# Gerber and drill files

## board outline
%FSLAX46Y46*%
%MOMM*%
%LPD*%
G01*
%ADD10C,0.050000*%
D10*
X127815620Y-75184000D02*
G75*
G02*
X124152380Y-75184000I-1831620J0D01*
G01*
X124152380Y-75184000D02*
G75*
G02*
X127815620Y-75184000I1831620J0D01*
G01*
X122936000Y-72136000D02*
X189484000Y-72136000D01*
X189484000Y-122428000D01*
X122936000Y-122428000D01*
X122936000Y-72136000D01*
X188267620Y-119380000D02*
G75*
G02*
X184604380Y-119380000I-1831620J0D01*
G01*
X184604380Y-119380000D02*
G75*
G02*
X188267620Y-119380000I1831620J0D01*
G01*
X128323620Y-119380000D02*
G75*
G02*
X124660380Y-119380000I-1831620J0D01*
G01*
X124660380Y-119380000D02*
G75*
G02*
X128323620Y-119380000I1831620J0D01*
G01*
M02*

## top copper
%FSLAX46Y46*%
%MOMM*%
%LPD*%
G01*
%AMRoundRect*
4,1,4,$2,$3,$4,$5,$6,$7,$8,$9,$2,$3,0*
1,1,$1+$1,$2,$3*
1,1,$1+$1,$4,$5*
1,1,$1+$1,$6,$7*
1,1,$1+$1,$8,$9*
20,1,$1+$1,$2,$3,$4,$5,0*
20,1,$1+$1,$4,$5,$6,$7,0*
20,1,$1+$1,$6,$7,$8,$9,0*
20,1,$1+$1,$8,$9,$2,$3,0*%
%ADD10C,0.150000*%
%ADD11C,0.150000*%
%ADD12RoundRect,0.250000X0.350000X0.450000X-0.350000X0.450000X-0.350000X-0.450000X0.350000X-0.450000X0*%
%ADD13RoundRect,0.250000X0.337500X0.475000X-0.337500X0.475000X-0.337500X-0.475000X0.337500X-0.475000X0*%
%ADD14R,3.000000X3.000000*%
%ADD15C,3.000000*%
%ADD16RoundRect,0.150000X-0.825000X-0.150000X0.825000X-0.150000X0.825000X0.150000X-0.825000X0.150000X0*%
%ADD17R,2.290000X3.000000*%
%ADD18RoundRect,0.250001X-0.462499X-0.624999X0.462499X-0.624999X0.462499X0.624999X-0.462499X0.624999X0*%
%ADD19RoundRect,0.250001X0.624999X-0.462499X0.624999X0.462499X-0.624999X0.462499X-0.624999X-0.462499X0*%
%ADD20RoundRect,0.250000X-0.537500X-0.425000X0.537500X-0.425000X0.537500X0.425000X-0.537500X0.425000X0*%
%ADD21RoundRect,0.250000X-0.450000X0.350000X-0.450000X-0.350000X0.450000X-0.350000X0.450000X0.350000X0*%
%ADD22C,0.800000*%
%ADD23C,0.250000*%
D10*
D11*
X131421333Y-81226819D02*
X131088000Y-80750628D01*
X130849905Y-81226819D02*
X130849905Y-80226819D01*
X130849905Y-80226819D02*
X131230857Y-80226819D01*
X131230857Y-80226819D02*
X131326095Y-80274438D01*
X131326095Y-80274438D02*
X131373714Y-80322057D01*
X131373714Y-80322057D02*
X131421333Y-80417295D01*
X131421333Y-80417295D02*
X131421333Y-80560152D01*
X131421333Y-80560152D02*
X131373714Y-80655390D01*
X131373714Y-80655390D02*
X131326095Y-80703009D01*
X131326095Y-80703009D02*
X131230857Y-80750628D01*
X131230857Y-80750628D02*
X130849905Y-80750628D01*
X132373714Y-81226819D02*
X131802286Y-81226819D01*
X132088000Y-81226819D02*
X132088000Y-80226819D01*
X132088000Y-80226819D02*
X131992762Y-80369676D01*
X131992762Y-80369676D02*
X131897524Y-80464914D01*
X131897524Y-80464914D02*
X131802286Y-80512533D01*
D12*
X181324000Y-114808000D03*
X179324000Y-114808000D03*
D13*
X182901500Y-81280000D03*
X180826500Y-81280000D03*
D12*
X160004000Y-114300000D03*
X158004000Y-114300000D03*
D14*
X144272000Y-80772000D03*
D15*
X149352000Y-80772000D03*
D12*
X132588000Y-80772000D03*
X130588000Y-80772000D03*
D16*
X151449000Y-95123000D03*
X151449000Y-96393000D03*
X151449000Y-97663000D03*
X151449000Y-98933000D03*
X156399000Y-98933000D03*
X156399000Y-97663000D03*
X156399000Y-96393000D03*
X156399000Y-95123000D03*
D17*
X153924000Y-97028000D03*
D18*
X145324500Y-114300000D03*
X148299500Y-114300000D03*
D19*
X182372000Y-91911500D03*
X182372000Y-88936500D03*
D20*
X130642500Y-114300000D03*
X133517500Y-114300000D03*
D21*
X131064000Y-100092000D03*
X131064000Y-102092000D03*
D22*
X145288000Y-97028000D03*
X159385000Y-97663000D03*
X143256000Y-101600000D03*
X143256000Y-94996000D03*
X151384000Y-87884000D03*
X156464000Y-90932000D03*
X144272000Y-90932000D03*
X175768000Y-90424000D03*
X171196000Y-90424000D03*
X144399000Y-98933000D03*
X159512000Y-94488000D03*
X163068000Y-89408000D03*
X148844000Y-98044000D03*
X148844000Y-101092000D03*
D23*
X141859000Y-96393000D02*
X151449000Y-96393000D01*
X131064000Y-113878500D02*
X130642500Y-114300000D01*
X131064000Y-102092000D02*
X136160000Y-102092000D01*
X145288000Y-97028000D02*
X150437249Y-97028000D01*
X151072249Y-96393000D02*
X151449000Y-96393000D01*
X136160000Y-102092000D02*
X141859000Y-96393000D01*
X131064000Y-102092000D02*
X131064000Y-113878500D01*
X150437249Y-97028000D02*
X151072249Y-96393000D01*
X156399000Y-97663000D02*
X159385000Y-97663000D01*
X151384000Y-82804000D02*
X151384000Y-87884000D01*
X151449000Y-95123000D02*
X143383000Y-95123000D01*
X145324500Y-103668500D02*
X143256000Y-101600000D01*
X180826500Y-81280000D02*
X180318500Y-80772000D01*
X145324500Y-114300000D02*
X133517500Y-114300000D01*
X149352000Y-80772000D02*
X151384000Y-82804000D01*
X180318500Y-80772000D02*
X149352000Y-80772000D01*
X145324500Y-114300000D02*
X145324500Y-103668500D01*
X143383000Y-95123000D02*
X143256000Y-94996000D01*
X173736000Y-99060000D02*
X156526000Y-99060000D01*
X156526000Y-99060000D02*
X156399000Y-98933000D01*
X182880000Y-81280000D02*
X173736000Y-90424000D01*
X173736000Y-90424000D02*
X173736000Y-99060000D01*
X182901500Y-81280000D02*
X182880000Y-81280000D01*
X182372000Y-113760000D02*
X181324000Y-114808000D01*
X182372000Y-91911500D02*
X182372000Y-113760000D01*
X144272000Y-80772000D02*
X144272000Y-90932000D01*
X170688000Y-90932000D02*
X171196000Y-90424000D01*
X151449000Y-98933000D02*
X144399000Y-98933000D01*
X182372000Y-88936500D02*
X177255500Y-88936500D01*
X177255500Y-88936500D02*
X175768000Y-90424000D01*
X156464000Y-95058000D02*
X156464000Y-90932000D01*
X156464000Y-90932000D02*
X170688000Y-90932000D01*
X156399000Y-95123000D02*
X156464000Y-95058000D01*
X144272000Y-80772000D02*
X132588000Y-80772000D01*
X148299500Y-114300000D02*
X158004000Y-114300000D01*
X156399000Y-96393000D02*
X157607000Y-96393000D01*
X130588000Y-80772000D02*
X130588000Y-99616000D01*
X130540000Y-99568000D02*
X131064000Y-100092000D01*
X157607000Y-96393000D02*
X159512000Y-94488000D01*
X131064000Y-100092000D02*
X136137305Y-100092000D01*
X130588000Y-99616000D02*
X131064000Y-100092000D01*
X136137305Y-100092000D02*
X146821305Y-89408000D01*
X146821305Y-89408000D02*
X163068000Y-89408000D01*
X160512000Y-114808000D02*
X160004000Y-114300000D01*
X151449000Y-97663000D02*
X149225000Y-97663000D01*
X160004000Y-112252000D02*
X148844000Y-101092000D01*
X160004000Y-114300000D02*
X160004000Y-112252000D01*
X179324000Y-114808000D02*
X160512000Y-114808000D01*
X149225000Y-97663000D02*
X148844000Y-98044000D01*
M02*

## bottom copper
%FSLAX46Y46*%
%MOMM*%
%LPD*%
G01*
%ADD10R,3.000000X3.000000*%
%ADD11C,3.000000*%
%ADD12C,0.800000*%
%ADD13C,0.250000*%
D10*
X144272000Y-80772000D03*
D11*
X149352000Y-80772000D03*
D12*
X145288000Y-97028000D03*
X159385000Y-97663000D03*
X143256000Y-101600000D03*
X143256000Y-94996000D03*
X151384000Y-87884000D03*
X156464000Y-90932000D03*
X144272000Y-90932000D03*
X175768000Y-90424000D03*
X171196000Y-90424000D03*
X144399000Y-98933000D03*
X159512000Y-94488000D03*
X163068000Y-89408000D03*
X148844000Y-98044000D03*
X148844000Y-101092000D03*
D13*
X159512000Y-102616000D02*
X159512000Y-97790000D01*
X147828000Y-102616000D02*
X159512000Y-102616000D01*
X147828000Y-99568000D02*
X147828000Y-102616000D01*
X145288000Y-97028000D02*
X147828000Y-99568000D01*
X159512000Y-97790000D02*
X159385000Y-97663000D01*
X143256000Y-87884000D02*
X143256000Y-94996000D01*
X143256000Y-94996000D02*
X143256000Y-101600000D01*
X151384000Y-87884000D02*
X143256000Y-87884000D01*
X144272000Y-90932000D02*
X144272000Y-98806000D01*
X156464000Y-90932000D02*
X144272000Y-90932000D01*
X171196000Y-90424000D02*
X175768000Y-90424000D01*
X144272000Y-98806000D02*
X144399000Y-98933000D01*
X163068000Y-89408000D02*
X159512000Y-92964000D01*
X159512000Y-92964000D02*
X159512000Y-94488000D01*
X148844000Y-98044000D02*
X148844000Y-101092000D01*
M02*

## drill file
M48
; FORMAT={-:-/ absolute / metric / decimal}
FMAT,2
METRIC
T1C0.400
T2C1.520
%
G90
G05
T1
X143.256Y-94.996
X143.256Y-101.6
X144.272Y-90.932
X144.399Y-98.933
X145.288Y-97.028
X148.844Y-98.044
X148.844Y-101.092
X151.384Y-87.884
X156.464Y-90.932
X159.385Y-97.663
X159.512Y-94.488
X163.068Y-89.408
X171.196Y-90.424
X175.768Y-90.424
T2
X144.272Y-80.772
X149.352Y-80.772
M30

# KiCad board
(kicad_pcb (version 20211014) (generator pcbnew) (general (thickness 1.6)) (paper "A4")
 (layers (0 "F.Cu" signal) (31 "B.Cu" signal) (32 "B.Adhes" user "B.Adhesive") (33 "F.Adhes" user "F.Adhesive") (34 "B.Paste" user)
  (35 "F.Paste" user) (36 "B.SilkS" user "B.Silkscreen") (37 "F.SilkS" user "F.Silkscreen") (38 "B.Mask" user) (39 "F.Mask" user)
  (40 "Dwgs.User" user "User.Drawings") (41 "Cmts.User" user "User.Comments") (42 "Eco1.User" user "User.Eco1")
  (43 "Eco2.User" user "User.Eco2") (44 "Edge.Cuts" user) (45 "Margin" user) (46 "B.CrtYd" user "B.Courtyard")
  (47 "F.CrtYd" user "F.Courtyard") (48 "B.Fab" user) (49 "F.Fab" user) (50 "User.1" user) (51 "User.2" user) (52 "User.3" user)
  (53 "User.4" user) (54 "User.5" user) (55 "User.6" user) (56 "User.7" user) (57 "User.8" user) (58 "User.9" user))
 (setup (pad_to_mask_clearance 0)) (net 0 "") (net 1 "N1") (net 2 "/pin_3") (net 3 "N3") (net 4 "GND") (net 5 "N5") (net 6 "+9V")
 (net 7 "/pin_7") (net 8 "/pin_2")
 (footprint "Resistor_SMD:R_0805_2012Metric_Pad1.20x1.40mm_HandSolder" (layer "F.Cu") (at 180.324 114.808 180)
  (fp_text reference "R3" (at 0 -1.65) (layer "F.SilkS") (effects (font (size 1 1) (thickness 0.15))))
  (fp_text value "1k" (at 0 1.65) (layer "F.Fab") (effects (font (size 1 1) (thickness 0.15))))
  (pad "1" smd roundrect (at -1 0 180) (size 1.2 1.4) (layers "F.Cu" "F.Paste" "F.Mask") (roundrect_rratio 0.208333) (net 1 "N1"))
  (pad "2" smd roundrect (at 1 0 180) (size 1.2 1.4) (layers "F.Cu" "F.Paste" "F.Mask") (roundrect_rratio 0.208333) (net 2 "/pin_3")))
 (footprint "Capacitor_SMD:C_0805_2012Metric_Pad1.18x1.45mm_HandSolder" (layer "F.Cu") (at 181.864 81.28 180)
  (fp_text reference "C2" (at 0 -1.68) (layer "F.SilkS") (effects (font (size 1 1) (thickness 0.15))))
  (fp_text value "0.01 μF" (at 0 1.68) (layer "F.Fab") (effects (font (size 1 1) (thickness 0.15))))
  (pad "1" smd roundrect (at -1.0375 0 180) (size 1.175 1.45) (layers "F.Cu" "F.Paste" "F.Mask") (roundrect_rratio 0.212766) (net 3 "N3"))
  (pad "2" smd roundrect (at 1.0375 0 180) (size 1.175 1.45) (layers "F.Cu" "F.Paste" "F.Mask") (roundrect_rratio 0.212766) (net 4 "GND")))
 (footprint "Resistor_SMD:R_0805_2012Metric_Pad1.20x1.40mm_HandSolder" (layer "F.Cu") (at 159.004 114.3 180)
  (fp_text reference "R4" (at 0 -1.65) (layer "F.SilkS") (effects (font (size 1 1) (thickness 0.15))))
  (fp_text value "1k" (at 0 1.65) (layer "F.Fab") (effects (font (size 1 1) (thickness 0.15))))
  (pad "1" smd roundrect (at -1 0 180) (size 1.2 1.4) (layers "F.Cu" "F.Paste" "F.Mask") (roundrect_rratio 0.208333) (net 2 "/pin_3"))
  (pad "2" smd roundrect (at 1 0 180) (size 1.2 1.4) (layers "F.Cu" "F.Paste" "F.Mask") (roundrect_rratio 0.208333) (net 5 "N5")))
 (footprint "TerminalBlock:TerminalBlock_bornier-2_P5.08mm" (layer "F.Cu") (at 144.272 80.772)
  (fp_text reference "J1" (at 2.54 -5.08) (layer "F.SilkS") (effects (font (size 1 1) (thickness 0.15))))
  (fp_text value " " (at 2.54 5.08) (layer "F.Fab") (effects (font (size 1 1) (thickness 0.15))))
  (pad "1" thru_hole rect (at 0 0) (size 3 3) (drill 1.52) (layers *.Cu *.Mask) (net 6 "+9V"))
  (pad "2" thru_hole circle (at 5.08 0) (size 3 3) (drill 1.52) (layers *.Cu *.Mask) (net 4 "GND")))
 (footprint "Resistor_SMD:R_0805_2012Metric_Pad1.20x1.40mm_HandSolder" (layer "F.Cu") (at 131.588 80.772 180)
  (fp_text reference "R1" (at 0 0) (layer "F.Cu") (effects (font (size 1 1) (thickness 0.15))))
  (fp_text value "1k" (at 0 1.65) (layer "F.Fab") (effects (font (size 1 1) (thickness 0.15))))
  (pad "1" smd roundrect (at -1 0 180) (size 1.2 1.4) (layers "F.Cu" "F.Paste" "F.Mask") (roundrect_rratio 0.208333) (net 6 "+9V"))
  (pad "2" smd roundrect (at 1 0 180) (size 1.2 1.4) (layers "F.Cu" "F.Paste" "F.Mask") (roundrect_rratio 0.208333) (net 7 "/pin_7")))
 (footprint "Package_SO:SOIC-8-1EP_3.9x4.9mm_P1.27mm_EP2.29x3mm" (layer "F.Cu") (at 153.924 97.028)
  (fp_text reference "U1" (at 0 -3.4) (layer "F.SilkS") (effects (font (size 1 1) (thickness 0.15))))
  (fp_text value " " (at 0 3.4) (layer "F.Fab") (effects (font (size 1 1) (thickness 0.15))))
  (pad "" smd roundrect (at -0.57 0.75) (size 0.92 1.21) (layers "F.Paste") (roundrect_rratio 0.25))
  (pad "" smd roundrect (at 0.57 -0.75) (size 0.92 1.21) (layers "F.Paste") (roundrect_rratio 0.25))
  (pad "" smd roundrect (at -0.57 -0.75) (size 0.92 1.21) (layers "F.Paste") (roundrect_rratio 0.25))
  (pad "" smd roundrect (at 0.57 0.75) (size 0.92 1.21) (layers "F.Paste") (roundrect_rratio 0.25))
  (pad "1" smd roundrect (at -2.475 -1.905) (size 1.95 0.6) (layers "F.Cu" "F.Paste" "F.Mask") (roundrect_rratio 0.25) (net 4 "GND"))
  (pad "2" smd roundrect (at -2.475 -0.635) (size 1.95 0.6) (layers "F.Cu" "F.Paste" "F.Mask") (roundrect_rratio 0.25) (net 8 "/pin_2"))
  (pad "3" smd roundrect (at -2.475 0.635) (size 1.95 0.6) (layers "F.Cu" "F.Paste" "F.Mask") (roundrect_rratio 0.25) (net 2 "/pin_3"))
  (pad "4" smd roundrect (at -2.475 1.905) (size 1.95 0.6) (layers "F.Cu" "F.Paste" "F.Mask") (roundrect_rratio 0.25) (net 6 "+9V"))
  (pad "5" smd roundrect (at 2.475 1.905) (size 1.95 0.6) (layers "F.Cu" "F.Paste" "F.Mask") (roundrect_rratio 0.25) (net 3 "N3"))
  (pad "6" smd roundrect (at 2.475 0.635) (size 1.95 0.6) (layers "F.Cu" "F.Paste" "F.Mask") (roundrect_rratio 0.25) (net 8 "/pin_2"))
  (pad "7" smd roundrect (at 2.475 -0.635) (size 1.95 0.6) (layers "F.Cu" "F.Paste" "F.Mask") (roundrect_rratio 0.25) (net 7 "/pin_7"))
  (pad "8" smd roundrect (at 2.475 -1.905) (size 1.95 0.6) (layers "F.Cu" "F.Paste" "F.Mask") (roundrect_rratio 0.25) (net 6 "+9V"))
  (pad "9" smd rect (at 0 0) (size 2.29 3) (layers "F.Cu" "F.Mask")))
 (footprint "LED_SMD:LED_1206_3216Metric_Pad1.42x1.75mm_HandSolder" (layer "F.Cu") (at 146.812 114.3)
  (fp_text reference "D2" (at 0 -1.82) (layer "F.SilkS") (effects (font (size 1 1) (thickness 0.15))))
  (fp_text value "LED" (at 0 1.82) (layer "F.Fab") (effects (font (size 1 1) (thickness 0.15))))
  (pad "1" smd roundrect (at -1.4875 0) (size 1.425 1.75) (layers "F.Cu" "F.Paste" "F.Mask") (roundrect_rratio 0.175439) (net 4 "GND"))
  (pad "2" smd roundrect (at 1.4875 0) (size 1.425 1.75) (layers "F.Cu" "F.Paste" "F.Mask") (roundrect_rratio 0.175439) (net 5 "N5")))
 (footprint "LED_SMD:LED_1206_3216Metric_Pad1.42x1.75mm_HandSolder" (layer "F.Cu") (at 182.372 90.424 90)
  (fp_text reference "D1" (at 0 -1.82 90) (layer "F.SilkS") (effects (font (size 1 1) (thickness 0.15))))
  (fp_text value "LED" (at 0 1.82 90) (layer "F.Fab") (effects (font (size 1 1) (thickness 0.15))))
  (pad "1" smd roundrect (at -1.4875 0 90) (size 1.425 1.75) (layers "F.Cu" "F.Paste" "F.Mask") (roundrect_rratio 0.175439) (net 1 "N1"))
  (pad "2" smd roundrect (at 1.4875 0 90) (size 1.425 1.75) (layers "F.Cu" "F.Paste" "F.Mask") (roundrect_rratio 0.175439) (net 6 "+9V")))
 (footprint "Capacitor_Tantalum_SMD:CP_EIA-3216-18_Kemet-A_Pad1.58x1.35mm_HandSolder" (layer "F.Cu") (at 132.08 114.3)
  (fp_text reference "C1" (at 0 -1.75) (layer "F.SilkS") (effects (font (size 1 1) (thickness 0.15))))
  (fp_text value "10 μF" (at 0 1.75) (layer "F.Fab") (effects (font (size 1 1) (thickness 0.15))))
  (pad "1" smd roundrect (at -1.4375 0) (size 1.575 1.35) (layers "F.Cu" "F.Paste" "F.Mask") (roundrect_rratio 0.185185) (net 8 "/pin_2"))
  (pad "2" smd roundrect (at 1.4375 0) (size 1.575 1.35) (layers "F.Cu" "F.Paste" "F.Mask") (roundrect_rratio 0.185185) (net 4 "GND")))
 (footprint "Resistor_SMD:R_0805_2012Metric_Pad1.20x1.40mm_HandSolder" (layer "F.Cu") (at 131.064 101.092 -90)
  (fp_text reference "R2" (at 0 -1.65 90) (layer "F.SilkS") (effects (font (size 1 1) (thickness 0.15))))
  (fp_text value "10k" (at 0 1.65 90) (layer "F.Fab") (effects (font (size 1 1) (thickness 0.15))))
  (pad "1" smd roundrect (at -1 0 270) (size 1.2 1.4) (layers "F.Cu" "F.Paste" "F.Mask") (roundrect_rratio 0.208333) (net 7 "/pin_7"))
  (pad "2" smd roundrect (at 1 0 270) (size 1.2 1.4) (layers "F.Cu" "F.Paste" "F.Mask") (roundrect_rratio 0.208333) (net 8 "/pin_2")))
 (gr_circle (center 125.984 75.184) (end 127 76.708) (layer "Edge.Cuts") (width 0.05) (fill none))
 (gr_rect (start 122.936 72.136) (end 189.484 122.428) (layer "Edge.Cuts") (width 0.05) (fill none))
 (gr_circle (center 186.436 119.38) (end 187.452 120.904) (layer "Edge.Cuts") (width 0.05) (fill none))
 (gr_circle (center 126.492 119.38) (end 127.508 120.904) (layer "Edge.Cuts") (width 0.05) (fill none))
 (segment (start 141.859 96.393) (end 151.449 96.393) (width 0.25) (layer "F.Cu") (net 8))
 (segment (start 131.064 113.8785) (end 130.6425 114.3) (width 0.25) (layer "F.Cu") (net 8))
 (segment (start 131.064 102.092) (end 136.16 102.092) (width 0.25) (layer "F.Cu") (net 8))
 (segment (start 145.288 97.028) (end 150.437249 97.028) (width 0.25) (layer "F.Cu") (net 8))
 (segment (start 151.072249 96.393) (end 151.449 96.393) (width 0.25) (layer "F.Cu") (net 8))
 (segment (start 136.16 102.092) (end 141.859 96.393) (width 0.25) (layer "F.Cu") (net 8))
 (segment (start 131.064 102.092) (end 131.064 113.8785) (width 0.25) (layer "F.Cu") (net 8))
 (segment (start 150.437249 97.028) (end 151.072249 96.393) (width 0.25) (layer "F.Cu") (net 8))
 (segment (start 156.399 97.663) (end 159.385 97.663) (width 0.25) (layer "F.Cu") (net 8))
 (via (at 145.288 97.028) (size 0.8) (drill 0.4) (layers "F.Cu" "B.Cu") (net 8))
 (via (at 159.385 97.663) (size 0.8) (drill 0.4) (layers "F.Cu" "B.Cu") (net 8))
 (segment (start 159.512 102.616) (end 159.512 97.79) (width 0.25) (layer "B.Cu") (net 8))
 (segment (start 147.828 102.616) (end 159.512 102.616) (width 0.25) (layer "B.Cu") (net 8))
 (segment (start 147.828 99.568) (end 147.828 102.616) (width 0.25) (layer "B.Cu") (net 8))
 (segment (start 145.288 97.028) (end 147.828 99.568) (width 0.25) (layer "B.Cu") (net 8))
 (segment (start 159.512 97.79) (end 159.385 97.663) (width 0.25) (layer "B.Cu") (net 8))
 (segment (start 151.384 82.804) (end 151.384 87.884) (width 0.25) (layer "F.Cu") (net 4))
 (segment (start 151.449 95.123) (end 143.383 95.123) (width 0.25) (layer "F.Cu") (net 4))
 (segment (start 145.3245 103.6685) (end 143.256 101.6) (width 0.25) (layer "F.Cu") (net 4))
 (segment (start 180.8265 81.28) (end 180.3185 80.772) (width 0.25) (layer "F.Cu") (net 4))
 (segment (start 145.3245 114.3) (end 133.5175 114.3) (width 0.25) (layer "F.Cu") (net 4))
 (segment (start 149.352 80.772) (end 151.384 82.804) (width 0.25) (layer "F.Cu") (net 4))
 (segment (start 180.3185 80.772) (end 149.352 80.772) (width 0.25) (layer "F.Cu") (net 4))
 (segment (start 145.3245 114.3) (end 145.3245 103.6685) (width 0.25) (layer "F.Cu") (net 4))
 (segment (start 143.383 95.123) (end 143.256 94.996) (width 0.25) (layer "F.Cu") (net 4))
 (via (at 143.256 101.6) (size 0.8) (drill 0.4) (layers "F.Cu" "B.Cu") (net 4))
 (via (at 143.256 94.996) (size 0.8) (drill 0.4) (layers "F.Cu" "B.Cu") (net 4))
 (via (at 151.384 87.884) (size 0.8) (drill 0.4) (layers "F.Cu" "B.Cu") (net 4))
 (segment (start 143.256 87.884) (end 143.256 94.996) (width 0.25) (layer "B.Cu") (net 4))
 (segment (start 143.256 94.996) (end 143.256 101.6) (width 0.25) (layer "B.Cu") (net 4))
 (segment (start 151.384 87.884) (end 143.256 87.884) (width 0.25) (layer "B.Cu") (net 4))
 (segment (start 173.736 99.06) (end 156.526 99.06) (width 0.25) (layer "F.Cu") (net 3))
 (segment (start 156.526 99.06) (end 156.399 98.933) (width 0.25) (layer "F.Cu") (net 3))
 (segment (start 182.88 81.28) (end 173.736 90.424) (width 0.25) (layer "F.Cu") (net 3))
 (segment (start 173.736 90.424) (end 173.736 99.06) (width 0.25) (layer "F.Cu") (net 3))
 (segment (start 182.9015 81.28) (end 182.88 81.28) (width 0.25) (layer "F.Cu") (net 3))
 (segment (start 182.372 113.76) (end 181.324 114.808) (width 0.25) (layer "F.Cu") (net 1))
 (segment (start 182.372 91.9115) (end 182.372 113.76) (width 0.25) (layer "F.Cu") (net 1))
 (segment (start 144.272 80.772) (end 144.272 90.932) (width 0.25) (layer "F.Cu") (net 6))
 (segment (start 170.688 90.932) (end 171.196 90.424) (width 0.25) (layer "F.Cu") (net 6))
 (segment (start 151.449 98.933) (end 144.399 98.933) (width 0.25) (layer "F.Cu") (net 6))
 (segment (start 182.372 88.9365) (end 177.2555 88.9365) (width 0.25) (layer "F.Cu") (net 6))
 (segment (start 177.2555 88.9365) (end 175.768 90.424) (width 0.25) (layer "F.Cu") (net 6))
 (segment (start 156.464 95.058) (end 156.464 90.932) (width 0.25) (layer "F.Cu") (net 6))
 (segment (start 156.464 90.932) (end 170.688 90.932) (width 0.25) (layer "F.Cu") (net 6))
 (segment (start 156.399 95.123) (end 156.464 95.058) (width 0.25) (layer "F.Cu") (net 6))
 (segment (start 144.272 80.772) (end 132.588 80.772) (width 0.25) (layer "F.Cu") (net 6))
 (via (at 156.464 90.932) (size 0.8) (drill 0.4) (layers "F.Cu" "B.Cu") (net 6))
 (via (at 144.272 90.932) (size 0.8) (drill 0.4) (layers "F.Cu" "B.Cu") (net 6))
 (via (at 175.768 90.424) (size 0.8) (drill 0.4) (layers "F.Cu" "B.Cu") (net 6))
 (via (at 171.196 90.424) (size 0.8) (drill 0.4) (layers "F.Cu" "B.Cu") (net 6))
 (via (at 144.399 98.933) (size 0.8) (drill 0.4) (layers "F.Cu" "B.Cu") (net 6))
 (segment (start 144.272 90.932) (end 144.272 98.806) (width 0.25) (layer "B.Cu") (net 6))
 (segment (start 156.464 90.932) (end 144.272 90.932) (width 0.25) (layer "B.Cu") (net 6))
 (segment (start 171.196 90.424) (end 175.768 90.424) (width 0.25) (layer "B.Cu") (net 6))
 (segment (start 144.272 98.806) (end 144.399 98.933) (width 0.25) (layer "B.Cu") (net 6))
 (segment (start 148.2995 114.3) (end 158.004 114.3) (width 0.25) (layer "F.Cu") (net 5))
 (segment (start 156.399 96.393) (end 157.607 96.393) (width 0.25) (layer "F.Cu") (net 7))
 (segment (start 130.588 80.772) (end 130.588 99.616) (width 0.25) (layer "F.Cu") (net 7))
 (segment (start 130.54 99.568) (end 131.064 100.092) (width 0.25) (layer "F.Cu") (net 7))
 (segment (start 157.607 96.393) (end 159.512 94.488) (width 0.25) (layer "F.Cu") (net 7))
 (segment (start 131.064 100.092) (end 136.137305 100.092) (width 0.25) (layer "F.Cu") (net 7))
 (segment (start 130.588 99.616) (end 131.064 100.092) (width 0.25) (layer "F.Cu") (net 7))
 (segment (start 136.137305 100.092) (end 146.821305 89.408) (width 0.25) (layer "F.Cu") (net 7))
 (segment (start 146.821305 89.408) (end 163.068 89.408) (width 0.25) (layer "F.Cu") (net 7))
 (via (at 159.512 94.488) (size 0.8) (drill 0.4) (layers "F.Cu" "B.Cu") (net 7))
 (via (at 163.068 89.408) (size 0.8) (drill 0.4) (layers "F.Cu" "B.Cu") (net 7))
 (segment (start 163.068 89.408) (end 159.512 92.964) (width 0.25) (layer "B.Cu") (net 7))
 (segment (start 159.512 92.964) (end 159.512 94.488) (width 0.25) (layer "B.Cu") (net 7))
 (segment (start 160.512 114.808) (end 160.004 114.3) (width 0.25) (layer "F.Cu") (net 2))
 (segment (start 151.449 97.663) (end 149.225 97.663) (width 0.25) (layer "F.Cu") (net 2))
 (segment (start 160.004 112.252) (end 148.844 101.092) (width 0.25) (layer "F.Cu") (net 2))
 (segment (start 160.004 114.3) (end 160.004 112.252) (width 0.25) (layer "F.Cu") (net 2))
 (segment (start 179.324 114.808) (end 160.512 114.808) (width 0.25) (layer "F.Cu") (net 2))
 (segment (start 149.225 97.663) (end 148.844 98.044) (width 0.25) (layer "F.Cu") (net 2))
 (via (at 148.844 98.044) (size 0.8) (drill 0.4) (layers "F.Cu" "B.Cu") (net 2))
 (via (at 148.844 101.092) (size 0.8) (drill 0.4) (layers "F.Cu" "B.Cu") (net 2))
 (segment (start 148.844 98.044) (end 148.844 101.092) (width 0.25) (layer "B.Cu") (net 2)))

